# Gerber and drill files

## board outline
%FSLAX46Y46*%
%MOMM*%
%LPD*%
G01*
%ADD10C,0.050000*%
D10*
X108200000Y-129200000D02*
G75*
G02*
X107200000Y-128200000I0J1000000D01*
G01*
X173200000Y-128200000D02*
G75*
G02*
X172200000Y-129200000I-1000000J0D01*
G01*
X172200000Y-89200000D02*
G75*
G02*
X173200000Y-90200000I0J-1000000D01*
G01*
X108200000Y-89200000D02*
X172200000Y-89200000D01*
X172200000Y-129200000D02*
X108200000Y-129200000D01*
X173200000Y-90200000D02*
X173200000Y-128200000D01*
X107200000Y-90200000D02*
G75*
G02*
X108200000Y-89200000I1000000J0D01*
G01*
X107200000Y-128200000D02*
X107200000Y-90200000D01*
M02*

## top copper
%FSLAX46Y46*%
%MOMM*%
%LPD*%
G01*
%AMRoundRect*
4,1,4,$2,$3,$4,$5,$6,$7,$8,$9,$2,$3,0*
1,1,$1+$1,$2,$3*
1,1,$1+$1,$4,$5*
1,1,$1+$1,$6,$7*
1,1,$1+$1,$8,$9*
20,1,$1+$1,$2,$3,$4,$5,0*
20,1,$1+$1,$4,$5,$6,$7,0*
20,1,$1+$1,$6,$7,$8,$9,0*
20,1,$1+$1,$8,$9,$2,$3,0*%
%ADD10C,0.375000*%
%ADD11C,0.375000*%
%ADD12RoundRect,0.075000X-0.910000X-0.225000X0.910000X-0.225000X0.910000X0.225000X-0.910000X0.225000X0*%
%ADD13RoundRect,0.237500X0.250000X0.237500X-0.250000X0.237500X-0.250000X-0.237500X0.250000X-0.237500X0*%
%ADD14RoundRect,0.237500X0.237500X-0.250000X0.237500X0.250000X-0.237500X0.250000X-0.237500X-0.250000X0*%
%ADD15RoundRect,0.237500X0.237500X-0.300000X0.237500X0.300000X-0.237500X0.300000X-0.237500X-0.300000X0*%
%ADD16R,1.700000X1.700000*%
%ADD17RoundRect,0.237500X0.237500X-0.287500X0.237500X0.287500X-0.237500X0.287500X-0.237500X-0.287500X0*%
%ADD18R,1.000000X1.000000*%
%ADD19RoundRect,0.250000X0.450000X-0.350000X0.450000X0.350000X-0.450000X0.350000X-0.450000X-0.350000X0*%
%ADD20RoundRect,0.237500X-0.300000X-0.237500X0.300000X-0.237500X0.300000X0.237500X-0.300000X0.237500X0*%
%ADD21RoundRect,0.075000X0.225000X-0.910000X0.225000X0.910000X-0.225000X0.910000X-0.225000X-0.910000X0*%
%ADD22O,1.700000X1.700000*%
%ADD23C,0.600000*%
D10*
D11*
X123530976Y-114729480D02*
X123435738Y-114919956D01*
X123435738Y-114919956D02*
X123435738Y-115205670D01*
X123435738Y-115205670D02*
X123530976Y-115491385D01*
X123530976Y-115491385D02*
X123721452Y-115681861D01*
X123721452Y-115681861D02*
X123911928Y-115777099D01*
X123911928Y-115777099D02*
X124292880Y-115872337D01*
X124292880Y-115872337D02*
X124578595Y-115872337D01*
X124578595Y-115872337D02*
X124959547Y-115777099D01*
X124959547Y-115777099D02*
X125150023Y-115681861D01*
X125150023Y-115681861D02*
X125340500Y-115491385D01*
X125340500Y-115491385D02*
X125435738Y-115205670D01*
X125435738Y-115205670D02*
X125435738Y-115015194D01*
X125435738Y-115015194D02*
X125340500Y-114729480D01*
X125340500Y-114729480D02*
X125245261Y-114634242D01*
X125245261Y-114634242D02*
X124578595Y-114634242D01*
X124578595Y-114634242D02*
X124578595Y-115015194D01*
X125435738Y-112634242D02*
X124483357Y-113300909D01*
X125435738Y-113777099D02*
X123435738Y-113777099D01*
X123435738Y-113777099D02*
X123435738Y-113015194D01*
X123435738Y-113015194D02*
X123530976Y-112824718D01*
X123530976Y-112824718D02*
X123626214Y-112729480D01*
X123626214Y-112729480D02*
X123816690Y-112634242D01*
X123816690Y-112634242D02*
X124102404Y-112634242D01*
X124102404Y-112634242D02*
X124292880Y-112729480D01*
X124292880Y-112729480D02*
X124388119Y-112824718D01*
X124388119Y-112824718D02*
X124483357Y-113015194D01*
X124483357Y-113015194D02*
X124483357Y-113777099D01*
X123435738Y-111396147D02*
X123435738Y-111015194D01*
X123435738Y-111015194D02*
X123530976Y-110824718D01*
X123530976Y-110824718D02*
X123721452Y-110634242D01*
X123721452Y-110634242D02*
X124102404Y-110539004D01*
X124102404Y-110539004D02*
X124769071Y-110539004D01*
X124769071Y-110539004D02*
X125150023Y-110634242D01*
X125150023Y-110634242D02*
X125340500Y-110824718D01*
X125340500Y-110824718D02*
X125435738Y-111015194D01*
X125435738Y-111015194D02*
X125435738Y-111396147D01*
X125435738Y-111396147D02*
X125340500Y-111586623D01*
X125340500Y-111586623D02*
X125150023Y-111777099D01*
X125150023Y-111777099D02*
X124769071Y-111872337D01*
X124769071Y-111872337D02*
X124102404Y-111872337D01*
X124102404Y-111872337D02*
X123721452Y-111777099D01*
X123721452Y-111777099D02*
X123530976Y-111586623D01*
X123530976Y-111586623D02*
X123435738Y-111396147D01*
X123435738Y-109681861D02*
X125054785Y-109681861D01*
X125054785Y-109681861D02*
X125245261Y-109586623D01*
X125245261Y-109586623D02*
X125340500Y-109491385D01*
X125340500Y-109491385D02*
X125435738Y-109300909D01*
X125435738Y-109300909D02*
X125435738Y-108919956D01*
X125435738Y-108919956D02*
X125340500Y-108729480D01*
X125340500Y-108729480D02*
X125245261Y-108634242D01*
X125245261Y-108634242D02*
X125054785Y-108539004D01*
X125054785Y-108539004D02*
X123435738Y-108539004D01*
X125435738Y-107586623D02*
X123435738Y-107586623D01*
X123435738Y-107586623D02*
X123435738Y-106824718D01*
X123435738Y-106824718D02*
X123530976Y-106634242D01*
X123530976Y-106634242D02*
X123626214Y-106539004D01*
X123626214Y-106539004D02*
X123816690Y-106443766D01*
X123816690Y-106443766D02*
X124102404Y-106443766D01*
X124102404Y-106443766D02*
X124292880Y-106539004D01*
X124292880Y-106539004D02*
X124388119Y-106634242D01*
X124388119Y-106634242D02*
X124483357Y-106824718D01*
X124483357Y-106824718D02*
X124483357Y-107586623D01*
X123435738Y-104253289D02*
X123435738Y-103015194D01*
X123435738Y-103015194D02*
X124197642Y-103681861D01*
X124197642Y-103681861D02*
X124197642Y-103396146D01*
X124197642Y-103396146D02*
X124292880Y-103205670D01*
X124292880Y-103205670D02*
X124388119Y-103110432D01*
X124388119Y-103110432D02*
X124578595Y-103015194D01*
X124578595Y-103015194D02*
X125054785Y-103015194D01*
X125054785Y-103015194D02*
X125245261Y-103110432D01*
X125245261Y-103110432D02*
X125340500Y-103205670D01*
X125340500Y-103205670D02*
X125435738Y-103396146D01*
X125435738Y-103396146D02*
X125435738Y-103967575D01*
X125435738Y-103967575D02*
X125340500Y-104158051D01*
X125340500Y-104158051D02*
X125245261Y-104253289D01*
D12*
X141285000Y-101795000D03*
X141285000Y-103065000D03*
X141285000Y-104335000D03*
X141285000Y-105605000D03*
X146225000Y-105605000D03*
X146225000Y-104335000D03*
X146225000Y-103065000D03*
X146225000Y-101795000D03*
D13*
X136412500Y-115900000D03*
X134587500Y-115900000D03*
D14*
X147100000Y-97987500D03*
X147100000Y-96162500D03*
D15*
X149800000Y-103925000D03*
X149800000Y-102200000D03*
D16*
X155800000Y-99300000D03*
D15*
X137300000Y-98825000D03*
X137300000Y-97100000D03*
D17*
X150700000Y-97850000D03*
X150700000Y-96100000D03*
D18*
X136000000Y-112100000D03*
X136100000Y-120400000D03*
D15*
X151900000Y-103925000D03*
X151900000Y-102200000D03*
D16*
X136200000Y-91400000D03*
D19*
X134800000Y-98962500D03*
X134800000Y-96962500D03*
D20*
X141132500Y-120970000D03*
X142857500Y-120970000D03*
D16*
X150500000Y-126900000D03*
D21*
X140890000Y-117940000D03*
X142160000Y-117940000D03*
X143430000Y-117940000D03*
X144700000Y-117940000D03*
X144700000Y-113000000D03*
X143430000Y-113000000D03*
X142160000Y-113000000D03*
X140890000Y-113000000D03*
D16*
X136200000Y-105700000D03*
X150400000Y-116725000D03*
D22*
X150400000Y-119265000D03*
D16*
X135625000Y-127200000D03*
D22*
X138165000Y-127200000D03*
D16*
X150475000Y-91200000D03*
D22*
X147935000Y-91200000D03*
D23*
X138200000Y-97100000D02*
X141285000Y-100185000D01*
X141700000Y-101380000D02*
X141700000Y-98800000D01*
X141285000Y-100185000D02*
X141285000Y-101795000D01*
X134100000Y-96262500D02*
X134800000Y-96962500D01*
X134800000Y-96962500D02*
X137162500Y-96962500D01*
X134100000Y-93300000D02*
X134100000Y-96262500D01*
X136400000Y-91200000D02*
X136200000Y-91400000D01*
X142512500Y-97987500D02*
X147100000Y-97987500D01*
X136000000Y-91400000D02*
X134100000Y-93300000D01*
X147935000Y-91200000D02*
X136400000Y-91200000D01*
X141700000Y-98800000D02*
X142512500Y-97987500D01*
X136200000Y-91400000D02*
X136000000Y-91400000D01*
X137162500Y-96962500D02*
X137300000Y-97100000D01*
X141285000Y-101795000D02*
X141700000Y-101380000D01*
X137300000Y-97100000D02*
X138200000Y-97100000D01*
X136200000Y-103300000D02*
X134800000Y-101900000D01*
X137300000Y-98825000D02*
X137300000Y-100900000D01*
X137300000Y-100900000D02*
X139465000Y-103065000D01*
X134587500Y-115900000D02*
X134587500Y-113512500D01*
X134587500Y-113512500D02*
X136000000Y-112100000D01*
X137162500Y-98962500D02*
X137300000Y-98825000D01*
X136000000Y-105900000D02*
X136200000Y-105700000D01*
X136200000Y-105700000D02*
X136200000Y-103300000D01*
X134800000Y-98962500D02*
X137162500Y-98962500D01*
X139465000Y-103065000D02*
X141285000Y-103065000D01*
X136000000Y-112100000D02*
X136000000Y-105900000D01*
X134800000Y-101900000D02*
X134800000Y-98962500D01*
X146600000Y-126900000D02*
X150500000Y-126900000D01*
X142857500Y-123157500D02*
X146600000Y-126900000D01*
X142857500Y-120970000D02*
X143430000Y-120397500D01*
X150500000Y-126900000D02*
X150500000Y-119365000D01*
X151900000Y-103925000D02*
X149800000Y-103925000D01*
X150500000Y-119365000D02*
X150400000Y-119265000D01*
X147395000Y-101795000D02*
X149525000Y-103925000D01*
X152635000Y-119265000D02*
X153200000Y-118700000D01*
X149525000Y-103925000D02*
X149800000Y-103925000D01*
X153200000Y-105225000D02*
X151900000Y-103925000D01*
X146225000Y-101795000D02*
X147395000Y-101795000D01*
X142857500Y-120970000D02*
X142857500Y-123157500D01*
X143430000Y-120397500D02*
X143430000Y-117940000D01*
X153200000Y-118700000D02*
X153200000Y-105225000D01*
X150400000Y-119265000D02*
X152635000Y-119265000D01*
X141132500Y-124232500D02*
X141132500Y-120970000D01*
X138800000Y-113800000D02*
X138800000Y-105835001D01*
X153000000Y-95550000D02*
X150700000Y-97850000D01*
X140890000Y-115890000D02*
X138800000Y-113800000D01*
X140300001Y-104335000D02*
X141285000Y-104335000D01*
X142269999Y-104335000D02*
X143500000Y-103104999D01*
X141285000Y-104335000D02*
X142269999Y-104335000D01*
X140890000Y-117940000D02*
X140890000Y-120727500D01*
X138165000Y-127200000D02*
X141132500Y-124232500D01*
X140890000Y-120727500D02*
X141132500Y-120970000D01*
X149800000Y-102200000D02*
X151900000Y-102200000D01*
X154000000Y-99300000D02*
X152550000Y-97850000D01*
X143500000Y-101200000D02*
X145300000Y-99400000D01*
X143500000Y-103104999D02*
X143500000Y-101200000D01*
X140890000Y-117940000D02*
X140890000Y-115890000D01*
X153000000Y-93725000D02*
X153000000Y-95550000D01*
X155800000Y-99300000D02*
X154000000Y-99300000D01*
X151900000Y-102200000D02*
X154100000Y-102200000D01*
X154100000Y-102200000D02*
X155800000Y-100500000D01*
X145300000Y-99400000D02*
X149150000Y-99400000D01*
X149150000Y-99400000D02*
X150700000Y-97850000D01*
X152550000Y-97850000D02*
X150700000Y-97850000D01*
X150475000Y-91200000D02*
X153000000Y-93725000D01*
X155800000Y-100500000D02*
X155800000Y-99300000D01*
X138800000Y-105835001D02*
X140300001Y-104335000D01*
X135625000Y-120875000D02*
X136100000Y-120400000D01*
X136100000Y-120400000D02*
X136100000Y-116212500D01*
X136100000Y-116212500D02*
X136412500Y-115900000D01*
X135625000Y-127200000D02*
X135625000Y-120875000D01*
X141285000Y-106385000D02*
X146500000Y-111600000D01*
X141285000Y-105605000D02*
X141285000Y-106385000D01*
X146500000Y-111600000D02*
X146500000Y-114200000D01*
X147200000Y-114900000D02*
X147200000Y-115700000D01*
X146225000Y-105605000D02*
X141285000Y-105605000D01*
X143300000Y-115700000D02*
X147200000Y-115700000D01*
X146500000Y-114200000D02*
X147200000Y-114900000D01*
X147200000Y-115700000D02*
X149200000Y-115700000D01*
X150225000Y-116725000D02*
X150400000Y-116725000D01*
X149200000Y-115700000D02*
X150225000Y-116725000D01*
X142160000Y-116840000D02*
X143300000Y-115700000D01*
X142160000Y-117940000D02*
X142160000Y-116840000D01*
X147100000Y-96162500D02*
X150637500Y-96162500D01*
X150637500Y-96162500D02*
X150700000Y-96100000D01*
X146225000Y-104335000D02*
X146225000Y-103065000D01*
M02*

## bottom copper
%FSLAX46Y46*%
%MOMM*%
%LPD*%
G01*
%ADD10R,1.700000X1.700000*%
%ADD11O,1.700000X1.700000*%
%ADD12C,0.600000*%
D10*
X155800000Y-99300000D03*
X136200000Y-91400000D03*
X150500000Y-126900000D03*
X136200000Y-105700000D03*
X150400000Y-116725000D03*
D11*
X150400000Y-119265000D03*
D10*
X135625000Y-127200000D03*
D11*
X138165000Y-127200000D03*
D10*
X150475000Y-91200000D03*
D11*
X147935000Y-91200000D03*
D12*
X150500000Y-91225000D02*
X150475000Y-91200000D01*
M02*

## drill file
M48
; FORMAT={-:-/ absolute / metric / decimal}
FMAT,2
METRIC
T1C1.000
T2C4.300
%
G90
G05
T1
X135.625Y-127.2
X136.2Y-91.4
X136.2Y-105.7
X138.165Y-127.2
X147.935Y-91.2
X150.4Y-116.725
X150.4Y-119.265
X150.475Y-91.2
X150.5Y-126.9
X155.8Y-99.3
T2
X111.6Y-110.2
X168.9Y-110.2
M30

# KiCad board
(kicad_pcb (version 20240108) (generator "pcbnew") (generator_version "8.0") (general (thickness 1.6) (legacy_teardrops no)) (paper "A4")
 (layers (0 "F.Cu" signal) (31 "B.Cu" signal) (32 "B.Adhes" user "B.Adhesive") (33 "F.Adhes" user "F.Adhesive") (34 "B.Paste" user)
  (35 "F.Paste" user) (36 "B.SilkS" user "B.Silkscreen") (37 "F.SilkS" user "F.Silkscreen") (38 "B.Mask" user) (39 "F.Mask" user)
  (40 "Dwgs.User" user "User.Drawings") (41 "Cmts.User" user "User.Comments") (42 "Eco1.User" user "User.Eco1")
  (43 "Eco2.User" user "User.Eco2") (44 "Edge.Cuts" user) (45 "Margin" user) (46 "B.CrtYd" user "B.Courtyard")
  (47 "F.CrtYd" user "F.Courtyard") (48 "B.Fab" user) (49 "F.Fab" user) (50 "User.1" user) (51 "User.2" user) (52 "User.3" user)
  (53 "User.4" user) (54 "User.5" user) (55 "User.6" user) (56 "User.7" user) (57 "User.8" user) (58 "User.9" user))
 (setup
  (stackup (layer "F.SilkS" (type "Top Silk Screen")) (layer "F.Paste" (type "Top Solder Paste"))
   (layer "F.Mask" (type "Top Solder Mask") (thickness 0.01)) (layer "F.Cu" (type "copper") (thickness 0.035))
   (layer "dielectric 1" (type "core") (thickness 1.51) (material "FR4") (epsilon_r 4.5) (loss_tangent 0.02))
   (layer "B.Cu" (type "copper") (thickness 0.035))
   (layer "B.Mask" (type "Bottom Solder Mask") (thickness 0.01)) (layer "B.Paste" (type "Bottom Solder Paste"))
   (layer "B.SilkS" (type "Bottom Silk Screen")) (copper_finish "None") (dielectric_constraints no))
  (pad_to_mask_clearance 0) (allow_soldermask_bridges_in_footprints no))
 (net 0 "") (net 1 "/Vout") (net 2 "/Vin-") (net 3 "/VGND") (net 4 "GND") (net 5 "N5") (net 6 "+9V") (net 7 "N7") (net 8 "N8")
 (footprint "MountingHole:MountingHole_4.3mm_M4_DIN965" (layer "F.Cu") (at 111.6 110.2 90)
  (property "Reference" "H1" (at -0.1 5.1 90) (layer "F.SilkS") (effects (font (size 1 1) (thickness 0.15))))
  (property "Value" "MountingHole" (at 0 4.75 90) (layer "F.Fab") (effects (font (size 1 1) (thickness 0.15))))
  (pad "" np_thru_hole circle (at 0 0 90) (size 4.3 4.3) (drill 4.3) (layers "*.Cu" "*.Mask")))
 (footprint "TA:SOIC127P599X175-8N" (layer "F.Cu") (at 143.755 103.7)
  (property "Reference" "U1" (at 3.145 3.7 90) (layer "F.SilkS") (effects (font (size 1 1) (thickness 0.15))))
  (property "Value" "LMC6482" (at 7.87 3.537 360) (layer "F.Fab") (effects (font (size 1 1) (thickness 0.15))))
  (pad "1" smd roundrect (at -2.47 -1.905) (size 1.97 0.6) (layers "F.Cu" "F.Paste" "F.Mask") (roundrect_rratio 0.125) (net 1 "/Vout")
   (solder_mask_margin 0.102))
  (pad "2" smd roundrect (at -2.47 -0.635) (size 1.97 0.6) (layers "F.Cu" "F.Paste" "F.Mask") (roundrect_rratio 0.125) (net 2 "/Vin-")
   (solder_mask_margin 0.102))
  (pad "3" smd roundrect (at -2.47 0.635) (size 1.97 0.6) (layers "F.Cu" "F.Paste" "F.Mask") (roundrect_rratio 0.125) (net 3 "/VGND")
   (solder_mask_margin 0.102))
  (pad "4" smd roundrect (at -2.47 1.905) (size 1.97 0.6) (layers "F.Cu" "F.Paste" "F.Mask") (roundrect_rratio 0.125) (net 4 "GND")
   (solder_mask_margin 0.102))
  (pad "5" smd roundrect (at 2.47 1.905) (size 1.97 0.6) (layers "F.Cu" "F.Paste" "F.Mask") (roundrect_rratio 0.125) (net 4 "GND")
   (solder_mask_margin 0.102))
  (pad "6" smd roundrect (at 2.47 0.635) (size 1.97 0.6) (layers "F.Cu" "F.Paste" "F.Mask") (roundrect_rratio 0.125) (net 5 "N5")
   (solder_mask_margin 0.102))
  (pad "7" smd roundrect (at 2.47 -0.635) (size 1.97 0.6) (layers "F.Cu" "F.Paste" "F.Mask") (roundrect_rratio 0.125) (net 5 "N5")
   (solder_mask_margin 0.102))
  (pad "8" smd roundrect (at 2.47 -1.905) (size 1.97 0.6) (layers "F.Cu" "F.Paste" "F.Mask") (roundrect_rratio 0.125) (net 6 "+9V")
   (solder_mask_margin 0.102)))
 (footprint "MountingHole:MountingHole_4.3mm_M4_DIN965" (layer "F.Cu") (at 168.9 110.2 90)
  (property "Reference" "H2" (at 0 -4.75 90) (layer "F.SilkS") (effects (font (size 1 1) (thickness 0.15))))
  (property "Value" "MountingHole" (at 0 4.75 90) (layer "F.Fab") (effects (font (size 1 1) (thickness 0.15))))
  (pad "" np_thru_hole circle (at 0 0 90) (size 4.3 4.3) (drill 4.3) (layers "*.Cu" "*.Mask")))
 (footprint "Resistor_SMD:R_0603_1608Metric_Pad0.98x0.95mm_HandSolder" (layer "F.Cu") (at 135.5 115.9 180)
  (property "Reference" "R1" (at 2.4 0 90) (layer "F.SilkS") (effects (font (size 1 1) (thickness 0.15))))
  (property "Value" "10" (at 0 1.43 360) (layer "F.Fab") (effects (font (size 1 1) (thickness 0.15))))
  (pad "1" smd roundrect (at -0.9125 0 180) (size 0.975 0.95) (layers "F.Cu" "F.Paste" "F.Mask") (roundrect_rratio 0.25) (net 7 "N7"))
  (pad "2" smd roundrect (at 0.9125 0 180) (size 0.975 0.95) (layers "F.Cu" "F.Paste" "F.Mask") (roundrect_rratio 0.25) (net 2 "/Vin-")))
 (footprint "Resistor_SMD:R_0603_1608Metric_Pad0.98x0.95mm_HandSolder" (layer "F.Cu") (at 147.1 97.075 90)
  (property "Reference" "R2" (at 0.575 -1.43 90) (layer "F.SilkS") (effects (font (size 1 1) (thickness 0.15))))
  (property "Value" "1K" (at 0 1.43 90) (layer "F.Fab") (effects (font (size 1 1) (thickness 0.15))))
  (pad "1" smd roundrect (at -0.9125 0 90) (size 0.975 0.95) (layers "F.Cu" "F.Paste" "F.Mask") (roundrect_rratio 0.25) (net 1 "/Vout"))
  (pad "2" smd roundrect (at 0.9125 0 90) (size 0.975 0.95) (layers "F.Cu" "F.Paste" "F.Mask") (roundrect_rratio 0.25) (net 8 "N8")))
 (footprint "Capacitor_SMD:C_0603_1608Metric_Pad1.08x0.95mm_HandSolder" (layer "F.Cu") (at 149.8 103.0625 90)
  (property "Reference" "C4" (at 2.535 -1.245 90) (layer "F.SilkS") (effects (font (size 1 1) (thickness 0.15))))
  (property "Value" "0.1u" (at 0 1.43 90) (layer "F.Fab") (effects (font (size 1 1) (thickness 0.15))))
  (pad "1" smd roundrect (at -0.8625 0 90) (size 1.075 0.95) (layers "F.Cu" "F.Paste" "F.Mask") (roundrect_rratio 0.25) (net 6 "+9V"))
  (pad "2" smd roundrect (at 0.8625 0 90) (size 1.075 0.95) (layers "F.Cu" "F.Paste" "F.Mask") (roundrect_rratio 0.25) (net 3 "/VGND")))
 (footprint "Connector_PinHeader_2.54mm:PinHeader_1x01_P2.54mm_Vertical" (layer "F.Cu") (at 155.8 99.3 90)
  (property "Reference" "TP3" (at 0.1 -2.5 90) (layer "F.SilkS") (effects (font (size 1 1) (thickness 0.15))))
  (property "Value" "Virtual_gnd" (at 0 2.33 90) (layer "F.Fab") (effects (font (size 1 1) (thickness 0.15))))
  (pad "1" thru_hole rect (at 0 0 90) (size 1.7 1.7) (drill 1) (layers "*.Cu" "*.Mask") (remove_unused_layers no) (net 3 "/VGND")))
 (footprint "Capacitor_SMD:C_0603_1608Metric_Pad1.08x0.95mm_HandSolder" (layer "F.Cu") (at 137.3 97.9625 90)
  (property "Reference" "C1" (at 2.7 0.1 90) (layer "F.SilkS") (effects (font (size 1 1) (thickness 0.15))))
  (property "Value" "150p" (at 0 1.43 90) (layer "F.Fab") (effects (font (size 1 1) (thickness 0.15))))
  (pad "1" smd roundrect (at -0.8625 0 90) (size 1.075 0.95) (layers "F.Cu" "F.Paste" "F.Mask") (roundrect_rratio 0.25) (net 2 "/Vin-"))
  (pad "2" smd roundrect (at 0.8625 0 90) (size 1.075 0.95) (layers "F.Cu" "F.Paste" "F.Mask") (roundrect_rratio 0.25) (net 1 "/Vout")))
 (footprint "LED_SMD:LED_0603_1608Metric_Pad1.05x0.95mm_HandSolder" (layer "F.Cu") (at 150.7 96.975 90)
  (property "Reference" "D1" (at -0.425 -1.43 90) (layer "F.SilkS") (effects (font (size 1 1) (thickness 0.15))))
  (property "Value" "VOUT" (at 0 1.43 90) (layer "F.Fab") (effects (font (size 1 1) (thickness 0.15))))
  (pad "1" smd roundrect (at -0.875 0 90) (size 1.05 0.95) (layers "F.Cu" "F.Paste" "F.Mask") (roundrect_rratio 0.25) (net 3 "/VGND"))
  (pad "2" smd roundrect (at 0.875 0 90) (size 1.05 0.95) (layers "F.Cu" "F.Paste" "F.Mask") (roundrect_rratio 0.25) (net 8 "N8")))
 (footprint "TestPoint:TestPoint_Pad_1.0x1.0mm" (layer "F.Cu") (at 136 112.1 90)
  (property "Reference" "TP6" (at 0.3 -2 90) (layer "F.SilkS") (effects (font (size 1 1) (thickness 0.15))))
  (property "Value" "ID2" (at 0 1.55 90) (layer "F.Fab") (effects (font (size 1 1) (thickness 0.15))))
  (pad "1" smd rect (at 0 0 90) (size 1 1) (layers "F.Cu" "F.Mask") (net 2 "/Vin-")))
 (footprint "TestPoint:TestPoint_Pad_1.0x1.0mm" (layer "F.Cu") (at 136.1 120.4 90)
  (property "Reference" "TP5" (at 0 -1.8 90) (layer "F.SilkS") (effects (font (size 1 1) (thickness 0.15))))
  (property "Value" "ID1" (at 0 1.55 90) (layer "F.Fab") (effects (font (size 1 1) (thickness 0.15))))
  (pad "1" smd rect (at 0 0 90) (size 1 1) (layers "F.Cu" "F.Mask") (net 7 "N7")))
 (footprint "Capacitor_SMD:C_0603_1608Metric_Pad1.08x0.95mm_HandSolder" (layer "F.Cu") (at 151.9 103.0625 90)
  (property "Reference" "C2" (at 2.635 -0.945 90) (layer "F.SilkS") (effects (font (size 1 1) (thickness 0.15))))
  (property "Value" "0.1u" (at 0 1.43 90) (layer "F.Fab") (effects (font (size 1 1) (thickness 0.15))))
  (pad "1" smd roundrect (at -0.8625 0 90) (size 1.075 0.95) (layers "F.Cu" "F.Paste" "F.Mask") (roundrect_rratio 0.25) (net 6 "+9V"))
  (pad "2" smd roundrect (at 0.8625 0 90) (size 1.075 0.95) (layers "F.Cu" "F.Paste" "F.Mask") (roundrect_rratio 0.25) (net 3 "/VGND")))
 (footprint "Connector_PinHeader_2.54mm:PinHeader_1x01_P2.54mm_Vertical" (layer "F.Cu") (at 136.2 91.4 90)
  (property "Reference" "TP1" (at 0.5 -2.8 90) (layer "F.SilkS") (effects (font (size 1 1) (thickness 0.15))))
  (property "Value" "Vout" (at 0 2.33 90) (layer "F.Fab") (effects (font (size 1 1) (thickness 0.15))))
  (pad "1" thru_hole rect (at 0 0 90) (size 1.7 1.7) (drill 1) (layers "*.Cu" "*.Mask") (remove_unused_layers no) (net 1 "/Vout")))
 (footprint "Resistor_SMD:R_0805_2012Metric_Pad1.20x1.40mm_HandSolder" (layer "F.Cu") (at 134.8 97.9625 90)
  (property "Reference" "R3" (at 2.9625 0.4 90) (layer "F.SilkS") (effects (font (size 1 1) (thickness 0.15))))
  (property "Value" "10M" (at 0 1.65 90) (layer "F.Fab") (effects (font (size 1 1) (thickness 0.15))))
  (pad "1" smd roundrect (at -1 0 90) (size 1.2 1.4) (layers "F.Cu" "F.Paste" "F.Mask") (roundrect_rratio 0.208333) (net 2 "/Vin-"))
  (pad "2" smd roundrect (at 1 0 90) (size 1.2 1.4) (layers "F.Cu" "F.Paste" "F.Mask") (roundrect_rratio 0.208333) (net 1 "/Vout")))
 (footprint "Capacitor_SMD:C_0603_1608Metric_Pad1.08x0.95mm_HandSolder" (layer "F.Cu") (at 141.995 120.97)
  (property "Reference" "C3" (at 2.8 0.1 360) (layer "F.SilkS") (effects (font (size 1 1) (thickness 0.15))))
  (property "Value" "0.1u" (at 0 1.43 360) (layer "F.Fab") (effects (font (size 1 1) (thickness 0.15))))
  (pad "1" smd roundrect (at -0.8625 0) (size 1.075 0.95) (layers "F.Cu" "F.Paste" "F.Mask") (roundrect_rratio 0.25) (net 3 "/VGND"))
  (pad "2" smd roundrect (at 0.8625 0) (size 1.075 0.95) (layers "F.Cu" "F.Paste" "F.Mask") (roundrect_rratio 0.25) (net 6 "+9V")))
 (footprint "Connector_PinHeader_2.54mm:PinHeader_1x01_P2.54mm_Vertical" (layer "F.Cu") (at 150.5 126.9 90)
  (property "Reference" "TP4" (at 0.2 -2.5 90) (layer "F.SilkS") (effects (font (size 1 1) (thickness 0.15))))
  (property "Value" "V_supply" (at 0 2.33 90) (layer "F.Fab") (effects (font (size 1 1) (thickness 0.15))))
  (pad "1" thru_hole rect (at 0 0 90) (size 1.7 1.7) (drill 1) (layers "*.Cu" "*.Mask") (remove_unused_layers no) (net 6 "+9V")))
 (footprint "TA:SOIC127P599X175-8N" (layer "F.Cu") (at 142.795 115.47 90)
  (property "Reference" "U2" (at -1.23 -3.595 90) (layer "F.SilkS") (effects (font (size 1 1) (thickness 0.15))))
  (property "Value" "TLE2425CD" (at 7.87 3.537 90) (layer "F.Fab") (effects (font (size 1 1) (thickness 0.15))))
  (pad "1" smd roundrect (at -2.47 -1.905 90) (size 1.97 0.6) (layers "F.Cu" "F.Paste" "F.Mask") (roundrect_rratio 0.125) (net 3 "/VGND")
   (solder_mask_margin 0.102))
  (pad "2" smd roundrect (at -2.47 -0.635 90) (size 1.97 0.6) (layers "F.Cu" "F.Paste" "F.Mask") (roundrect_rratio 0.125) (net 4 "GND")
   (solder_mask_margin 0.102))
  (pad "3" smd roundrect (at -2.47 0.635 90) (size 1.97 0.6) (layers "F.Cu" "F.Paste" "F.Mask") (roundrect_rratio 0.125) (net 6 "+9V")
   (solder_mask_margin 0.102))
  (pad "4" smd roundrect (at -2.47 1.905 90) (size 1.97 0.6) (layers "F.Cu" "F.Paste" "F.Mask") (roundrect_rratio 0.125)
   (solder_mask_margin 0.102))
  (pad "5" smd roundrect (at 2.47 1.905 90) (size 1.97 0.6) (layers "F.Cu" "F.Paste" "F.Mask") (roundrect_rratio 0.125)
   (solder_mask_margin 0.102))
  (pad "6" smd roundrect (at 2.47 0.635 90) (size 1.97 0.6) (layers "F.Cu" "F.Paste" "F.Mask") (roundrect_rratio 0.125)
   (solder_mask_margin 0.102))
  (pad "7" smd roundrect (at 2.47 -0.635 90) (size 1.97 0.6) (layers "F.Cu" "F.Paste" "F.Mask") (roundrect_rratio 0.125)
   (solder_mask_margin 0.102))
  (pad "8" smd roundrect (at 2.47 -1.905 90) (size 1.97 0.6) (layers "F.Cu" "F.Paste" "F.Mask") (roundrect_rratio 0.125)
   (solder_mask_margin 0.102)))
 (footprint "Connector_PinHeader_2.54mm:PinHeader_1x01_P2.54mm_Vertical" (layer "F.Cu") (at 136.2 105.7 90)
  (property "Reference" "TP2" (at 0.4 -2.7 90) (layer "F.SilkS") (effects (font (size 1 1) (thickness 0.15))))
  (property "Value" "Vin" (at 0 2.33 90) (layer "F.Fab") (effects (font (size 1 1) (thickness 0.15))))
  (pad "1" thru_hole rect (at 0 0 90) (size 1.7 1.7) (drill 1) (layers "*.Cu" "*.Mask") (remove_unused_layers no) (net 2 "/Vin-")))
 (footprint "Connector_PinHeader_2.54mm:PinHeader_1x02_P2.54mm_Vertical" (layer "B.Cu") (at 150.4 116.725 180)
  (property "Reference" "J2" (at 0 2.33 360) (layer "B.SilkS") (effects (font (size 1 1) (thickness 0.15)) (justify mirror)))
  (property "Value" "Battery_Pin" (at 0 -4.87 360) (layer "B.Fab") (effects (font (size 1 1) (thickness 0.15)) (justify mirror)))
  (pad "1" thru_hole rect (at 0 0 180) (size 1.7 1.7) (drill 1) (layers "*.Cu" "*.Mask") (remove_unused_layers no) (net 4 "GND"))
  (pad "2" thru_hole oval (at 0 -2.54 180) (size 1.7 1.7) (drill 1) (layers "*.Cu" "*.Mask") (remove_unused_layers no) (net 6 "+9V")))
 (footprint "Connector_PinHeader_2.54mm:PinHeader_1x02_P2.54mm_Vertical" (layer "B.Cu") (at 135.625 127.2 -90)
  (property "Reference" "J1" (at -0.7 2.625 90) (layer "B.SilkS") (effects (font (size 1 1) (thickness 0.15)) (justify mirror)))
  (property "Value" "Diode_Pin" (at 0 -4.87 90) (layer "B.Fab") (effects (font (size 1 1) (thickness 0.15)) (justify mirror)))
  (pad "1" thru_hole rect (at 0 0 270) (size 1.7 1.7) (drill 1) (layers "*.Cu" "*.Mask") (remove_unused_layers no) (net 7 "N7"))
  (pad "2" thru_hole oval (at 0 -2.54 270) (size 1.7 1.7) (drill 1) (layers "*.Cu" "*.Mask") (remove_unused_layers no) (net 3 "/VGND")))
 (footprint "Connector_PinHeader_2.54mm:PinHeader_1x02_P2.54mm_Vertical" (layer "B.Cu") (at 150.475 91.2 90)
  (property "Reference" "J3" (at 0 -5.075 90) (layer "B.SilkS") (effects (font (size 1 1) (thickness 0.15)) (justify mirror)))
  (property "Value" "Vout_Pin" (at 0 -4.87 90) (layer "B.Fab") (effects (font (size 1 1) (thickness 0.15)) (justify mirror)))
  (pad "1" thru_hole rect (at 0 0 90) (size 1.7 1.7) (drill 1) (layers "*.Cu" "*.Mask") (remove_unused_layers no) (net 3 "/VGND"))
  (pad "2" thru_hole oval (at 0 -2.54 90) (size 1.7 1.7) (drill 1) (layers "*.Cu" "*.Mask") (remove_unused_layers no) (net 1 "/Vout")))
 (gr_arc (start 108.2 129.2) (mid 107.492893 128.907107) (end 107.2 128.2) (stroke (width 0.05) (type default)) (layer "Edge.Cuts"))
 (gr_arc (start 173.2 128.2) (mid 172.907107 128.907107) (end 172.2 129.2) (stroke (width 0.05) (type default)) (layer "Edge.Cuts"))
 (gr_arc (start 172.2 89.2) (mid 172.907107 89.492893) (end 173.2 90.2) (stroke (width 0.05) (type default)) (layer "Edge.Cuts"))
 (gr_line (start 108.2 89.2) (end 172.2 89.2) (stroke (width 0.05) (type default)) (layer "Edge.Cuts"))
 (gr_line (start 172.2 129.2) (end 108.2 129.2) (stroke (width 0.05) (type default)) (layer "Edge.Cuts"))
 (gr_line (start 173.2 90.2) (end 173.2 128.2) (stroke (width 0.05) (type default)) (layer "Edge.Cuts"))
 (gr_arc (start 107.2 90.2) (mid 107.492893 89.492893) (end 108.2 89.2) (stroke (width 0.05) (type default)) (layer "Edge.Cuts"))
 (gr_line (start 107.2 128.2) (end 107.2 90.2) (stroke (width 0.05) (type default)) (layer "Edge.Cuts"))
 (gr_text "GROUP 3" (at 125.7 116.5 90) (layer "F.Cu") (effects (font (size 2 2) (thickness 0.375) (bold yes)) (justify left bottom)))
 (segment (start 138.2 97.1) (end 141.285 100.185) (width 0.6) (layer "F.Cu") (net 1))
 (segment (start 141.7 101.38) (end 141.7 98.8) (width 0.6) (layer "F.Cu") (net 1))
 (segment (start 141.285 100.185) (end 141.285 101.795) (width 0.6) (layer "F.Cu") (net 1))
 (segment (start 134.1 96.2625) (end 134.8 96.9625) (width 0.6) (layer "F.Cu") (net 1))
 (segment (start 134.8 96.9625) (end 137.1625 96.9625) (width 0.6) (layer "F.Cu") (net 1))
 (segment (start 134.1 93.3) (end 134.1 96.2625) (width 0.6) (layer "F.Cu") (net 1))
 (segment (start 136.4 91.2) (end 136.2 91.4) (width 0.6) (layer "F.Cu") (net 1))
 (segment (start 142.5125 97.9875) (end 147.1 97.9875) (width 0.6) (layer "F.Cu") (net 1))
 (segment (start 136 91.4) (end 134.1 93.3) (width 0.6) (layer "F.Cu") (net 1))
 (segment (start 147.935 91.2) (end 136.4 91.2) (width 0.6) (layer "F.Cu") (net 1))
 (segment (start 141.7 98.8) (end 142.5125 97.9875) (width 0.6) (layer "F.Cu") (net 1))
 (segment (start 136.2 91.4) (end 136 91.4) (width 0.6) (layer "F.Cu") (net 1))
 (segment (start 137.1625 96.9625) (end 137.3 97.1) (width 0.6) (layer "F.Cu") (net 1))
 (segment (start 141.285 101.795) (end 141.7 101.38) (width 0.6) (layer "F.Cu") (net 1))
 (segment (start 137.3 97.1) (end 138.2 97.1) (width 0.6) (layer "F.Cu") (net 1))
 (segment (start 136.2 103.3) (end 134.8 101.9) (width 0.6) (layer "F.Cu") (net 2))
 (segment (start 137.3 98.825) (end 137.3 100.9) (width 0.6) (layer "F.Cu") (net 2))
 (segment (start 137.3 100.9) (end 139.465 103.065) (width 0.6) (layer "F.Cu") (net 2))
 (segment (start 134.5875 115.9) (end 134.5875 113.5125) (width 0.6) (layer "F.Cu") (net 2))
 (segment (start 134.5875 113.5125) (end 136 112.1) (width 0.6) (layer "F.Cu") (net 2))
 (segment (start 137.1625 98.9625) (end 137.3 98.825) (width 0.6) (layer "F.Cu") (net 2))
 (segment (start 136 105.9) (end 136.2 105.7) (width 0.6) (layer "F.Cu") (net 2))
 (segment (start 136.2 105.7) (end 136.2 103.3) (width 0.6) (layer "F.Cu") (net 2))
 (segment (start 134.8 98.9625) (end 137.1625 98.9625) (width 0.6) (layer "F.Cu") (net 2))
 (segment (start 139.465 103.065) (end 141.285 103.065) (width 0.6) (layer "F.Cu") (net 2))
 (segment (start 136 112.1) (end 136 105.9) (width 0.6) (layer "F.Cu") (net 2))
 (segment (start 134.8 101.9) (end 134.8 98.9625) (width 0.6) (layer "F.Cu") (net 2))
 (segment (start 146.6 126.9) (end 150.5 126.9) (width 0.6) (layer "F.Cu") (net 6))
 (segment (start 142.8575 123.1575) (end 146.6 126.9) (width 0.6) (layer "F.Cu") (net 6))
 (segment (start 142.8575 120.97) (end 143.43 120.3975) (width 0.6) (layer "F.Cu") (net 6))
 (segment (start 150.5 126.9) (end 150.5 119.365) (width 0.6) (layer "F.Cu") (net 6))
 (segment (start 151.9 103.925) (end 149.8 103.925) (width 0.6) (layer "F.Cu") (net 6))
 (segment (start 150.5 119.365) (end 150.4 119.265) (width 0.6) (layer "F.Cu") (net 6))
 (segment (start 147.395 101.795) (end 149.525 103.925) (width 0.6) (layer "F.Cu") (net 6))
 (segment (start 152.635 119.265) (end 153.2 118.7) (width 0.6) (layer "F.Cu") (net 6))
 (segment (start 149.525 103.925) (end 149.8 103.925) (width 0.6) (layer "F.Cu") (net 6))
 (segment (start 153.2 105.225) (end 151.9 103.925) (width 0.6) (layer "F.Cu") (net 6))
 (segment (start 146.225 101.795) (end 147.395 101.795) (width 0.6) (layer "F.Cu") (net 6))
 (segment (start 142.8575 120.97) (end 142.8575 123.1575) (width 0.6) (layer "F.Cu") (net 6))
 (segment (start 143.43 120.3975) (end 143.43 117.94) (width 0.6) (layer "F.Cu") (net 6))
 (segment (start 153.2 118.7) (end 153.2 105.225) (width 0.6) (layer "F.Cu") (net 6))
 (segment (start 150.4 119.265) (end 152.635 119.265) (width 0.6) (layer "F.Cu") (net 6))
 (segment (start 141.1325 124.2325) (end 141.1325 120.97) (width 0.6) (layer "F.Cu") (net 3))
 (segment (start 138.8 113.8) (end 138.8 105.835001) (width 0.6) (layer "F.Cu") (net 3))
 (segment (start 153 95.55) (end 150.7 97.85) (width 0.6) (layer "F.Cu") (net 3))
 (segment (start 140.89 115.89) (end 138.8 113.8) (width 0.6) (layer "F.Cu") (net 3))
 (segment (start 140.300001 104.335) (end 141.285 104.335) (width 0.6) (layer "F.Cu") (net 3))
 (segment (start 142.269999 104.335) (end 143.5 103.104999) (width 0.6) (layer "F.Cu") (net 3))
 (segment (start 141.285 104.335) (end 142.269999 104.335) (width 0.6) (layer "F.Cu") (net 3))
 (segment (start 140.89 117.94) (end 140.89 120.7275) (width 0.6) (layer "F.Cu") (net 3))
 (segment (start 138.165 127.2) (end 141.1325 124.2325) (width 0.6) (layer "F.Cu") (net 3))
 (segment (start 140.89 120.7275) (end 141.1325 120.97) (width 0.6) (layer "F.Cu") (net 3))
 (segment (start 149.8 102.2) (end 151.9 102.2) (width 0.6) (layer "F.Cu") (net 3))
 (segment (start 154 99.3) (end 152.55 97.85) (width 0.6) (layer "F.Cu") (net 3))
 (segment (start 143.5 101.2) (end 145.3 99.4) (width 0.6) (layer "F.Cu") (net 3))
 (segment (start 143.5 103.104999) (end 143.5 101.2) (width 0.6) (layer "F.Cu") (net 3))
 (segment (start 140.89 117.94) (end 140.89 115.89) (width 0.6) (layer "F.Cu") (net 3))
 (segment (start 153 93.725) (end 153 95.55) (width 0.6) (layer "F.Cu") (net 3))
 (segment (start 155.8 99.3) (end 154 99.3) (width 0.6) (layer "F.Cu") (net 3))
 (segment (start 151.9 102.2) (end 154.1 102.2) (width 0.6) (layer "F.Cu") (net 3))
 (segment (start 154.1 102.2) (end 155.8 100.5) (width 0.6) (layer "F.Cu") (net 3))
 (segment (start 145.3 99.4) (end 149.15 99.4) (width 0.6) (layer "F.Cu") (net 3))
 (segment (start 149.15 99.4) (end 150.7 97.85) (width 0.6) (layer "F.Cu") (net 3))
 (segment (start 152.55 97.85) (end 150.7 97.85) (width 0.6) (layer "F.Cu") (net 3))
 (segment (start 150.475 91.2) (end 153 93.725) (width 0.6) (layer "F.Cu") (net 3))
 (segment (start 155.8 100.5) (end 155.8 99.3) (width 0.6) (layer "F.Cu") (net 3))
 (segment (start 138.8 105.835001) (end 140.300001 104.335) (width 0.6) (layer "F.Cu") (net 3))
 (segment (start 150.5 91.225) (end 150.475 91.2) (width 0.6) (layer "B.Cu") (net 3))
 (segment (start 135.625 120.875) (end 136.1 120.4) (width 0.6) (layer "F.Cu") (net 7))
 (segment (start 136.1 120.4) (end 136.1 116.2125) (width 0.6) (layer "F.Cu") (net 7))
 (segment (start 136.1 116.2125) (end 136.4125 115.9) (width 0.6) (layer "F.Cu") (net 7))
 (segment (start 135.625 127.2) (end 135.625 120.875) (width 0.6) (layer "F.Cu") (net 7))
 (segment (start 141.285 106.385) (end 146.5 111.6) (width 0.6) (layer "F.Cu") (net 4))
 (segment (start 141.285 105.605) (end 141.285 106.385) (width 0.6) (layer "F.Cu") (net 4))
 (segment (start 146.5 111.6) (end 146.5 114.2) (width 0.6) (layer "F.Cu") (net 4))
 (segment (start 147.2 114.9) (end 147.2 115.7) (width 0.6) (layer "F.Cu") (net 4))
 (segment (start 146.225 105.605) (end 141.285 105.605) (width 0.6) (layer "F.Cu") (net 4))
 (segment (start 143.3 115.7) (end 147.2 115.7) (width 0.6) (layer "F.Cu") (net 4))
 (segment (start 146.5 114.2) (end 147.2 114.9) (width 0.6) (layer "F.Cu") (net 4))
 (segment (start 147.2 115.7) (end 149.2 115.7) (width 0.6) (layer "F.Cu") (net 4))
 (segment (start 150.225 116.725) (end 150.4 116.725) (width 0.6) (layer "F.Cu") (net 4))
 (segment (start 149.2 115.7) (end 150.225 116.725) (width 0.6) (layer "F.Cu") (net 4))
 (segment (start 142.16 116.84) (end 143.3 115.7) (width 0.6) (layer "F.Cu") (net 4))
 (segment (start 142.16 117.94) (end 142.16 116.84) (width 0.6) (layer "F.Cu") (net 4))
 (segment (start 147.1 96.1625) (end 150.6375 96.1625) (width 0.6) (layer "F.Cu") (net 8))
 (segment (start 150.6375 96.1625) (end 150.7 96.1) (width 0.6) (layer "F.Cu") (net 8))
 (segment (start 146.225 104.335) (end 146.225 103.065) (width 0.6) (layer "F.Cu") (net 5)))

